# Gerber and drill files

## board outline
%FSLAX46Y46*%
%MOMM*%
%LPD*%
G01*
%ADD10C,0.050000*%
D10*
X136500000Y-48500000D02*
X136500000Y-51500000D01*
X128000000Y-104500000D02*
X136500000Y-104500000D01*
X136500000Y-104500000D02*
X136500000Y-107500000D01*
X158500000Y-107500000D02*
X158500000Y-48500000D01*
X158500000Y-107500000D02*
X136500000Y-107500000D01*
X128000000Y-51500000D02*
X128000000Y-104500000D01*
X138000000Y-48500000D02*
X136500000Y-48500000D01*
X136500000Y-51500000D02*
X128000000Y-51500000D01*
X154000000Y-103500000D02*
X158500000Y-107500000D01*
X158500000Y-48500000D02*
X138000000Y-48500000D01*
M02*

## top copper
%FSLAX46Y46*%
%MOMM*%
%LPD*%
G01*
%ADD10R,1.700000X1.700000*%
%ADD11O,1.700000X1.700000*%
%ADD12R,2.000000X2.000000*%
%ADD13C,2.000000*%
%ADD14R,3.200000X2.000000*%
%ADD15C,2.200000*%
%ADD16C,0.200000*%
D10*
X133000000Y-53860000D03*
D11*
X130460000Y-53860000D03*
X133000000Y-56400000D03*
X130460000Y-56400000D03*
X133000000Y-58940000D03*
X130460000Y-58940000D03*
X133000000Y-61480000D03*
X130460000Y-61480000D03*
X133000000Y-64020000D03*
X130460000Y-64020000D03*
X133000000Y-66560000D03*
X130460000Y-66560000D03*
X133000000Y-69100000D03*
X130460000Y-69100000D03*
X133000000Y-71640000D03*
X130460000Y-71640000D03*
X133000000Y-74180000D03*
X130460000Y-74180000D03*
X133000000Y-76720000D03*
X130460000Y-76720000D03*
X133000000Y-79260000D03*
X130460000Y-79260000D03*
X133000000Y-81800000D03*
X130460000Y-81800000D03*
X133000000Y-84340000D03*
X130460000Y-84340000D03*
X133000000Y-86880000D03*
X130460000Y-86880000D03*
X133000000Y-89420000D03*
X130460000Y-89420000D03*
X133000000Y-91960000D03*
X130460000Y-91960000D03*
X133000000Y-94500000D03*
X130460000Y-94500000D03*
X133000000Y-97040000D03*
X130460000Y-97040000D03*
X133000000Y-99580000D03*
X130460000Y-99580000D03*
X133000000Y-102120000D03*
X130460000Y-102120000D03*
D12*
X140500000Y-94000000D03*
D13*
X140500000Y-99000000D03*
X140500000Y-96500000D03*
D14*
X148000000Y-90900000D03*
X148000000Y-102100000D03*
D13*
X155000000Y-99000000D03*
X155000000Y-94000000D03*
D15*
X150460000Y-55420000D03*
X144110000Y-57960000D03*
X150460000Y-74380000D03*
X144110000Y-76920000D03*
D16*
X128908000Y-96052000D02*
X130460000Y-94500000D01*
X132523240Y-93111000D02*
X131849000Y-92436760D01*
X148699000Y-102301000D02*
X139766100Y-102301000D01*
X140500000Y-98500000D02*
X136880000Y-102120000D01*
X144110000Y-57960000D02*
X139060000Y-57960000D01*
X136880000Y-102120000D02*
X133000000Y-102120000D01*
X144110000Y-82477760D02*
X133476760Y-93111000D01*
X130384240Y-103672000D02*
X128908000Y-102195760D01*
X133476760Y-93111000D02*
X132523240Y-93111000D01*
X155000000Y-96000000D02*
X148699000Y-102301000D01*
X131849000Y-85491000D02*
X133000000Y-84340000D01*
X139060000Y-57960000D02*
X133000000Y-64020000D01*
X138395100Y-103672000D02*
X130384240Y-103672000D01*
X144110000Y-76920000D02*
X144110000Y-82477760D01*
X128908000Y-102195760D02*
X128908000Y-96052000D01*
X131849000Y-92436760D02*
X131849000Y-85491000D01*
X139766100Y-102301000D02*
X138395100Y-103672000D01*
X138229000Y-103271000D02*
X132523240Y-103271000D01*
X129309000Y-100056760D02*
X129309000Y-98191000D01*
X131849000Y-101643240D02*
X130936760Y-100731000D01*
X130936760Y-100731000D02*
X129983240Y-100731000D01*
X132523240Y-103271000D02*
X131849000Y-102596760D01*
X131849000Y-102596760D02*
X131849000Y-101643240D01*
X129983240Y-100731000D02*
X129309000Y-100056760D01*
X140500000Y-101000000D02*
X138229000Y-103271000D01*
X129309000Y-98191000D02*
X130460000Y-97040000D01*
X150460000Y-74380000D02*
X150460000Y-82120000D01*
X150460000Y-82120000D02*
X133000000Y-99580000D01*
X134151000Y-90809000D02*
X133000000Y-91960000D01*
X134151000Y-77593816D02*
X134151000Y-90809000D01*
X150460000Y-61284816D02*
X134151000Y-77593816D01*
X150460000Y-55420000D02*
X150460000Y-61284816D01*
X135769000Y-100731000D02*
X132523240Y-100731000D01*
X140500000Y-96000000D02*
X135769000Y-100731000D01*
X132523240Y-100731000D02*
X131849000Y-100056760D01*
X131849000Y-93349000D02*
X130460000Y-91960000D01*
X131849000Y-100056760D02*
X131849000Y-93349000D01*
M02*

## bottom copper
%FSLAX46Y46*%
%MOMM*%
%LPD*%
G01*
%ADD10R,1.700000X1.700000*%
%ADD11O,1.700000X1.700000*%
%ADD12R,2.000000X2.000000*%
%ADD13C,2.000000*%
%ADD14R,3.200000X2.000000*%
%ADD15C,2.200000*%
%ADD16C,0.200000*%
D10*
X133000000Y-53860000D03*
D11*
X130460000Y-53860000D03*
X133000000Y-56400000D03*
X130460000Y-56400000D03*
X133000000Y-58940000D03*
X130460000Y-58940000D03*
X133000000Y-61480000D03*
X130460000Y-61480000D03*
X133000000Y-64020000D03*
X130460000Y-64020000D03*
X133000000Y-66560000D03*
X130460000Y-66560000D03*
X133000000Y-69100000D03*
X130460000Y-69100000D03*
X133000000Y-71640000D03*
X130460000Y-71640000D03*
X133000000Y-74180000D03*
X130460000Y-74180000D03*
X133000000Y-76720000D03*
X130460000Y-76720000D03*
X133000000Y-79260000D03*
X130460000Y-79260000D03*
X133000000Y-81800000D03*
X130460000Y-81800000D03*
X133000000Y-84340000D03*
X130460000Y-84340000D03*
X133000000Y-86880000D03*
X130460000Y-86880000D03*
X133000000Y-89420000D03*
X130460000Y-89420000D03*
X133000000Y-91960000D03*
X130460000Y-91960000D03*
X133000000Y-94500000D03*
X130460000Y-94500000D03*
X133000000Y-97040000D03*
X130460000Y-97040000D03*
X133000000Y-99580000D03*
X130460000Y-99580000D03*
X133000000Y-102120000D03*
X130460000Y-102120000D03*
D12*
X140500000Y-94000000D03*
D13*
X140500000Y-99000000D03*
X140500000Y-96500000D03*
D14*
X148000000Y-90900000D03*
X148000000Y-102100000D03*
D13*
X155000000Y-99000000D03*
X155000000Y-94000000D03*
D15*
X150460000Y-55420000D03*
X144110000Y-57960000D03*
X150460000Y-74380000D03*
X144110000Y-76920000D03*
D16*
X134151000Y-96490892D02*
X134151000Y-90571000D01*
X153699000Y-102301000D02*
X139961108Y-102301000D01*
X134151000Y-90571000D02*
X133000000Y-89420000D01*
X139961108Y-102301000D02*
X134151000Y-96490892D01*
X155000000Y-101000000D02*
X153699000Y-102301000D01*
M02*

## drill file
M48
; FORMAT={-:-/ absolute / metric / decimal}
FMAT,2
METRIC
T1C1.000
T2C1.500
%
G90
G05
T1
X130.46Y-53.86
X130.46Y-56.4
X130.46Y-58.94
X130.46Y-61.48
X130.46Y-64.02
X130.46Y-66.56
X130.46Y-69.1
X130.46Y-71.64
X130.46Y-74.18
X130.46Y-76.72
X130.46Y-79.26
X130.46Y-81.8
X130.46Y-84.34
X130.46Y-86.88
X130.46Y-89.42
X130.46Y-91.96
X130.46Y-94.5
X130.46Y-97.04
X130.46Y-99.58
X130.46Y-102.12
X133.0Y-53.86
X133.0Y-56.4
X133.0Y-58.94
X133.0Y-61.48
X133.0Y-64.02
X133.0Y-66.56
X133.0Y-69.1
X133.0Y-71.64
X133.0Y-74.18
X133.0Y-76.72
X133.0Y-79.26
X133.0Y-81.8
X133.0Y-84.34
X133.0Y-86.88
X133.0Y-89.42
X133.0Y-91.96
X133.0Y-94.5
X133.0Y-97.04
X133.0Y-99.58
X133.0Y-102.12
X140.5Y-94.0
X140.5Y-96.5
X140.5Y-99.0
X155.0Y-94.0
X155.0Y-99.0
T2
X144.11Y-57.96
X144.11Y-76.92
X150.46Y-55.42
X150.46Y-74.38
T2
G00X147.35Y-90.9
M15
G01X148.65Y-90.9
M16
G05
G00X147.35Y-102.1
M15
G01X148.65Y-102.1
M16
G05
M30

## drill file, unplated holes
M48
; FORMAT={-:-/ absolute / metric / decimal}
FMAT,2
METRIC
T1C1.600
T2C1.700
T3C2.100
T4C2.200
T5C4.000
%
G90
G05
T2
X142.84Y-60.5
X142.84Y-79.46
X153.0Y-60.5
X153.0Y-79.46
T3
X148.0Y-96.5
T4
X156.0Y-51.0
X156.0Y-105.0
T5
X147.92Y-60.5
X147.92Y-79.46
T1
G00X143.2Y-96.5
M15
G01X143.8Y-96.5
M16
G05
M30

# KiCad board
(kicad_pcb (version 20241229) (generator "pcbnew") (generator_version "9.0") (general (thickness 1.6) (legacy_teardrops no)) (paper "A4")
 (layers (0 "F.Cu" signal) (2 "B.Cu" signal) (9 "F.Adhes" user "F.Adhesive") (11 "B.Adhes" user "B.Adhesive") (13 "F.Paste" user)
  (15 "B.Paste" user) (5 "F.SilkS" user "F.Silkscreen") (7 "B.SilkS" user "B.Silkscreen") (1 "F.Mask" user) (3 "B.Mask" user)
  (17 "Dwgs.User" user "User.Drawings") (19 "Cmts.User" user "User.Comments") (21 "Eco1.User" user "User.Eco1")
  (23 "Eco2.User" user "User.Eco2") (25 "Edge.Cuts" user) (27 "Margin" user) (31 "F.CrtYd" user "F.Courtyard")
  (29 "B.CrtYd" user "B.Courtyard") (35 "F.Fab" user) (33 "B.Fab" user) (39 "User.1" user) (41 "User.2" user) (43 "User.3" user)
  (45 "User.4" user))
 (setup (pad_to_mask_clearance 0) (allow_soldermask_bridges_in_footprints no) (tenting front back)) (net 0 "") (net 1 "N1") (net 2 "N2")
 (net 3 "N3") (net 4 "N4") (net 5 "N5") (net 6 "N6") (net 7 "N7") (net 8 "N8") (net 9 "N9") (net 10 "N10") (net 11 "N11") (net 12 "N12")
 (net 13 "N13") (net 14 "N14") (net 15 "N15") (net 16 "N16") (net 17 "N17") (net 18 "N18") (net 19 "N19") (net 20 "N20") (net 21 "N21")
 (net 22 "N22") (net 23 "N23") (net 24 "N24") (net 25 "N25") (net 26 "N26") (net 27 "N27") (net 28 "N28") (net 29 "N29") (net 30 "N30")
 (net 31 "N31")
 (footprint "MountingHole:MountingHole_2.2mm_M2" (layer "F.Cu") (at 156 105)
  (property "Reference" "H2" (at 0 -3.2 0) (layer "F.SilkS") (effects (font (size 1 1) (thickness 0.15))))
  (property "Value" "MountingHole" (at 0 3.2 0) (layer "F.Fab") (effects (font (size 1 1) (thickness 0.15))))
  (pad "" np_thru_hole circle (at 0 0) (size 2.2 2.2) (drill 2.2) (layers "*.Cu" "*.Mask")))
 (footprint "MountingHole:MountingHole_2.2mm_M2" (layer "F.Cu") (at 156 51)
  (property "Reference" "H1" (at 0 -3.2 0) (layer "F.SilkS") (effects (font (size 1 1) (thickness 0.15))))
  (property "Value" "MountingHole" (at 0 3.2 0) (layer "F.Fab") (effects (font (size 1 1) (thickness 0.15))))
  (pad "" np_thru_hole circle (at 0 0) (size 2.2 2.2) (drill 2.2) (layers "*.Cu" "*.Mask")))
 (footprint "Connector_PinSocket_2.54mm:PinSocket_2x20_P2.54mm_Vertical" (layer "F.Cu") (at 133 53.86)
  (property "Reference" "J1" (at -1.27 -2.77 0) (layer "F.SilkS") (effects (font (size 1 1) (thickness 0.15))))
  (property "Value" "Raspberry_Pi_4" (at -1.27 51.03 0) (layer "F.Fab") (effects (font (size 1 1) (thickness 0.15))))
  (pad "1" thru_hole rect (at 0 0) (size 1.7 1.7) (drill 1) (layers "*.Cu" "*.Mask") (remove_unused_layers no) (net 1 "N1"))
  (pad "2" thru_hole oval (at -2.54 0) (size 1.7 1.7) (drill 1) (layers "*.Cu" "*.Mask") (remove_unused_layers no) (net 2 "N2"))
  (pad "3" thru_hole oval (at 0 2.54) (size 1.7 1.7) (drill 1) (layers "*.Cu" "*.Mask") (remove_unused_layers no) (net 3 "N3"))
  (pad "4" thru_hole oval (at -2.54 2.54) (size 1.7 1.7) (drill 1) (layers "*.Cu" "*.Mask") (remove_unused_layers no) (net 2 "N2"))
  (pad "5" thru_hole oval (at 0 5.08) (size 1.7 1.7) (drill 1) (layers "*.Cu" "*.Mask") (remove_unused_layers no) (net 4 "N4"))
  (pad "6" thru_hole oval (at -2.54 5.08) (size 1.7 1.7) (drill 1) (layers "*.Cu" "*.Mask") (remove_unused_layers no) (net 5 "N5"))
  (pad "7" thru_hole oval (at 0 7.62) (size 1.7 1.7) (drill 1) (layers "*.Cu" "*.Mask") (remove_unused_layers no) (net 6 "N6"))
  (pad "8" thru_hole oval (at -2.54 7.62) (size 1.7 1.7) (drill 1) (layers "*.Cu" "*.Mask") (remove_unused_layers no) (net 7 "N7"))
  (pad "9" thru_hole oval (at 0 10.16) (size 1.7 1.7) (drill 1) (layers "*.Cu" "*.Mask") (remove_unused_layers no) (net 5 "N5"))
  (pad "10" thru_hole oval (at -2.54 10.16) (size 1.7 1.7) (drill 1) (layers "*.Cu" "*.Mask") (remove_unused_layers no) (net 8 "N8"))
  (pad "11" thru_hole oval (at 0 12.7) (size 1.7 1.7) (drill 1) (layers "*.Cu" "*.Mask") (remove_unused_layers no) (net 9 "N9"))
  (pad "12" thru_hole oval (at -2.54 12.7) (size 1.7 1.7) (drill 1) (layers "*.Cu" "*.Mask") (remove_unused_layers no) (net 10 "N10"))
  (pad "13" thru_hole oval (at 0 15.24) (size 1.7 1.7) (drill 1) (layers "*.Cu" "*.Mask") (remove_unused_layers no) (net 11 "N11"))
  (pad "14" thru_hole oval (at -2.54 15.24) (size 1.7 1.7) (drill 1) (layers "*.Cu" "*.Mask") (remove_unused_layers no) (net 5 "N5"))
  (pad "15" thru_hole oval (at 0 17.78) (size 1.7 1.7) (drill 1) (layers "*.Cu" "*.Mask") (remove_unused_layers no) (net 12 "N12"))
  (pad "16" thru_hole oval (at -2.54 17.78) (size 1.7 1.7) (drill 1) (layers "*.Cu" "*.Mask") (remove_unused_layers no) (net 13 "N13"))
  (pad "17" thru_hole oval (at 0 20.32) (size 1.7 1.7) (drill 1) (layers "*.Cu" "*.Mask") (remove_unused_layers no) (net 1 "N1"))
  (pad "18" thru_hole oval (at -2.54 20.32) (size 1.7 1.7) (drill 1) (layers "*.Cu" "*.Mask") (remove_unused_layers no) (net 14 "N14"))
  (pad "19" thru_hole oval (at 0 22.86) (size 1.7 1.7) (drill 1) (layers "*.Cu" "*.Mask") (remove_unused_layers no) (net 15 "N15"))
  (pad "20" thru_hole oval (at -2.54 22.86) (size 1.7 1.7) (drill 1) (layers "*.Cu" "*.Mask") (remove_unused_layers no) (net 5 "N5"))
  (pad "21" thru_hole oval (at 0 25.4) (size 1.7 1.7) (drill 1) (layers "*.Cu" "*.Mask") (remove_unused_layers no) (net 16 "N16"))
  (pad "22" thru_hole oval (at -2.54 25.4) (size 1.7 1.7) (drill 1) (layers "*.Cu" "*.Mask") (remove_unused_layers no) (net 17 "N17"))
  (pad "23" thru_hole oval (at 0 27.94) (size 1.7 1.7) (drill 1) (layers "*.Cu" "*.Mask") (remove_unused_layers no) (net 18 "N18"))
  (pad "24" thru_hole oval (at -2.54 27.94) (size 1.7 1.7) (drill 1) (layers "*.Cu" "*.Mask") (remove_unused_layers no) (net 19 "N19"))
  (pad "25" thru_hole oval (at 0 30.48) (size 1.7 1.7) (drill 1) (layers "*.Cu" "*.Mask") (remove_unused_layers no) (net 5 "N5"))
  (pad "26" thru_hole oval (at -2.54 30.48) (size 1.7 1.7) (drill 1) (layers "*.Cu" "*.Mask") (remove_unused_layers no) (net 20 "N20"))
  (pad "27" thru_hole oval (at 0 33.02) (size 1.7 1.7) (drill 1) (layers "*.Cu" "*.Mask") (remove_unused_layers no) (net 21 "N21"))
  (pad "28" thru_hole oval (at -2.54 33.02) (size 1.7 1.7) (drill 1) (layers "*.Cu" "*.Mask") (remove_unused_layers no) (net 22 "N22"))
  (pad "29" thru_hole oval (at 0 35.56) (size 1.7 1.7) (drill 1) (layers "*.Cu" "*.Mask") (remove_unused_layers no) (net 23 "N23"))
  (pad "30" thru_hole oval (at -2.54 35.56) (size 1.7 1.7) (drill 1) (layers "*.Cu" "*.Mask") (remove_unused_layers no) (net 5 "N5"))
  (pad "31" thru_hole oval (at 0 38.1) (size 1.7 1.7) (drill 1) (layers "*.Cu" "*.Mask") (remove_unused_layers no) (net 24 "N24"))
  (pad "32" thru_hole oval (at -2.54 38.1) (size 1.7 1.7) (drill 1) (layers "*.Cu" "*.Mask") (remove_unused_layers no) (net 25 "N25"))
  (pad "33" thru_hole oval (at 0 40.64) (size 1.7 1.7) (drill 1) (layers "*.Cu" "*.Mask") (remove_unused_layers no) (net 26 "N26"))
  (pad "34" thru_hole oval (at -2.54 40.64) (size 1.7 1.7) (drill 1) (layers "*.Cu" "*.Mask") (remove_unused_layers no) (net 5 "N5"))
  (pad "35" thru_hole oval (at 0 43.18) (size 1.7 1.7) (drill 1) (layers "*.Cu" "*.Mask") (remove_unused_layers no) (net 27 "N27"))
  (pad "36" thru_hole oval (at -2.54 43.18) (size 1.7 1.7) (drill 1) (layers "*.Cu" "*.Mask") (remove_unused_layers no) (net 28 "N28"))
  (pad "37" thru_hole oval (at 0 45.72) (size 1.7 1.7) (drill 1) (layers "*.Cu" "*.Mask") (remove_unused_layers no) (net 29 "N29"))
  (pad "38" thru_hole oval (at -2.54 45.72) (size 1.7 1.7) (drill 1) (layers "*.Cu" "*.Mask") (remove_unused_layers no) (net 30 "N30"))
  (pad "39" thru_hole oval (at 0 48.26) (size 1.7 1.7) (drill 1) (layers "*.Cu" "*.Mask") (remove_unused_layers no) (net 5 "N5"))
  (pad "40" thru_hole oval (at -2.54 48.26) (size 1.7 1.7) (drill 1) (layers "*.Cu" "*.Mask") (remove_unused_layers no) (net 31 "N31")))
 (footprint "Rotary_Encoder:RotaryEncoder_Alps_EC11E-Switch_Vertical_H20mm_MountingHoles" (layer "F.Cu") (at 140.5 94)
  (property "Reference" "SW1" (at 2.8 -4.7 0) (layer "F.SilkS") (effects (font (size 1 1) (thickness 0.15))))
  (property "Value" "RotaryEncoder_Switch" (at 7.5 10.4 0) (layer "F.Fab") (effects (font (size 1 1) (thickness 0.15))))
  (pad "" np_thru_hole oval (at 3 2.5) (size 2.2 1.6) (drill oval 2.2 1.6) (layers "*.Mask"))
  (pad "" np_thru_hole circle (at 7.5 2.5) (size 2.1 2.1) (drill 2.1) (layers "*.Mask"))
  (pad "A" thru_hole rect (at 0 0) (size 2 2) (drill 1) (layers "*.Cu" "*.Mask") (remove_unused_layers no) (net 25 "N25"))
  (pad "B" thru_hole circle (at 0 5) (size 2 2) (drill 1) (layers "*.Cu" "*.Mask") (remove_unused_layers no) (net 28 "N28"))
  (pad "C" thru_hole circle (at 0 2.5) (size 2 2) (drill 1) (layers "*.Cu" "*.Mask") (remove_unused_layers no) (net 5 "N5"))
  (pad "MP" thru_hole rect (at 7.5 -3.1) (size 3.2 2) (drill oval 2.8 1.5) (layers "*.Cu" "*.Mask") (remove_unused_layers no))
  (pad "MP" thru_hole rect (at 7.5 8.1) (size 3.2 2) (drill oval 2.8 1.5) (layers "*.Cu" "*.Mask") (remove_unused_layers no))
  (pad "S1" thru_hole circle (at 14.5 5) (size 2 2) (drill 1) (layers "*.Cu" "*.Mask") (remove_unused_layers no) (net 23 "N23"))
  (pad "S2" thru_hole circle (at 14.5 0) (size 2 2) (drill 1) (layers "*.Cu" "*.Mask") (remove_unused_layers no) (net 5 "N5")))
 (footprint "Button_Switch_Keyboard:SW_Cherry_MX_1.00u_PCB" (layer "F.Cu") (at 150.46 55.42)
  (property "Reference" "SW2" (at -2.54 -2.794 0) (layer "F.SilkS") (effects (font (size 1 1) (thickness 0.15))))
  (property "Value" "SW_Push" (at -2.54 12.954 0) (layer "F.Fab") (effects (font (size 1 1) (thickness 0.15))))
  (pad "" np_thru_hole circle (at -7.62 5.08) (size 1.7 1.7) (drill 1.7) (layers "*.Cu" "*.Mask"))
  (pad "" np_thru_hole circle (at -2.54 5.08) (size 4 4) (drill 4) (layers "*.Cu" "*.Mask"))
  (pad "" np_thru_hole circle (at 2.54 5.08) (size 1.7 1.7) (drill 1.7) (layers "*.Cu" "*.Mask"))
  (pad "1" thru_hole circle (at 0 0) (size 2.2 2.2) (drill 1.5) (layers "*.Cu" "*.Mask") (remove_unused_layers no) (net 24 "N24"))
  (pad "2" thru_hole circle (at -6.35 2.54) (size 2.2 2.2) (drill 1.5) (layers "*.Cu" "*.Mask") (remove_unused_layers no) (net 5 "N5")))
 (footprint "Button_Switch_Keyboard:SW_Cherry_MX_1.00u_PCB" (layer "F.Cu") (at 150.46 74.38)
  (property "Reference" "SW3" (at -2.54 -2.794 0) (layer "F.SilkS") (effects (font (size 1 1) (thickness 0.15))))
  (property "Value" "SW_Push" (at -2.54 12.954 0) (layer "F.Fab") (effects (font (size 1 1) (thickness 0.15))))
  (pad "" np_thru_hole circle (at -7.62 5.08) (size 1.7 1.7) (drill 1.7) (layers "*.Cu" "*.Mask"))
  (pad "" np_thru_hole circle (at -2.54 5.08) (size 4 4) (drill 4) (layers "*.Cu" "*.Mask"))
  (pad "" np_thru_hole circle (at 2.54 5.08) (size 1.7 1.7) (drill 1.7) (layers "*.Cu" "*.Mask"))
  (pad "1" thru_hole circle (at 0 0) (size 2.2 2.2) (drill 1.5) (layers "*.Cu" "*.Mask") (remove_unused_layers no) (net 29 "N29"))
  (pad "2" thru_hole circle (at -6.35 2.54) (size 2.2 2.2) (drill 1.5) (layers "*.Cu" "*.Mask") (remove_unused_layers no) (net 5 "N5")))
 (gr_line (start 136.5 48.5) (end 136.5 51.5) (stroke (width 0.05) (type default)) (layer "Edge.Cuts"))
 (gr_line (start 128 104.5) (end 136.5 104.5) (stroke (width 0.05) (type default)) (layer "Edge.Cuts"))
 (gr_line (start 136.5 104.5) (end 136.5 107.5) (stroke (width 0.05) (type default)) (layer "Edge.Cuts"))
 (gr_line (start 158.5 107.5) (end 158.5 48.5) (stroke (width 0.05) (type default)) (layer "Edge.Cuts"))
 (gr_line (start 158.5 107.5) (end 136.5 107.5) (stroke (width 0.05) (type default)) (layer "Edge.Cuts"))
 (gr_line (start 128 51.5) (end 128 104.5) (stroke (width 0.05) (type default)) (layer "Edge.Cuts"))
 (gr_line (start 138 48.5) (end 136.5 48.5) (stroke (width 0.05) (type default)) (layer "Edge.Cuts"))
 (gr_line (start 136.5 51.5) (end 128 51.5) (stroke (width 0.05) (type default)) (layer "Edge.Cuts"))
 (gr_line (start 154 103.5) (end 158.5 107.5) (stroke (width 0.05) (type default)) (layer "Edge.Cuts"))
 (gr_line (start 158.5 48.5) (end 138 48.5) (stroke (width 0.05) (type default)) (layer "Edge.Cuts"))
 (segment (start 134.151 96.490892) (end 134.151 90.571) (width 0.2) (layer "B.Cu") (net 23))
 (segment (start 153.699 102.301) (end 139.961108 102.301) (width 0.2) (layer "B.Cu") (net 23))
 (segment (start 134.151 90.571) (end 133 89.42) (width 0.2) (layer "B.Cu") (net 23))
 (segment (start 139.961108 102.301) (end 134.151 96.490892) (width 0.2) (layer "B.Cu") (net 23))
 (segment (start 155 101) (end 153.699 102.301) (width 0.2) (layer "B.Cu") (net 23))
 (segment (start 128.908 96.052) (end 130.46 94.5) (width 0.2) (layer "F.Cu") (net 5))
 (segment (start 132.52324 93.111) (end 131.849 92.43676) (width 0.2) (layer "F.Cu") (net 5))
 (segment (start 148.699 102.301) (end 139.7661 102.301) (width 0.2) (layer "F.Cu") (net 5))
 (segment (start 140.5 98.5) (end 136.88 102.12) (width 0.2) (layer "F.Cu") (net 5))
 (segment (start 144.11 57.96) (end 139.06 57.96) (width 0.2) (layer "F.Cu") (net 5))
 (segment (start 136.88 102.12) (end 133 102.12) (width 0.2) (layer "F.Cu") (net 5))
 (segment (start 144.11 82.47776) (end 133.47676 93.111) (width 0.2) (layer "F.Cu") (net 5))
 (segment (start 130.38424 103.672) (end 128.908 102.19576) (width 0.2) (layer "F.Cu") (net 5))
 (segment (start 133.47676 93.111) (end 132.52324 93.111) (width 0.2) (layer "F.Cu") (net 5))
 (segment (start 155 96) (end 148.699 102.301) (width 0.2) (layer "F.Cu") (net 5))
 (segment (start 131.849 85.491) (end 133 84.34) (width 0.2) (layer "F.Cu") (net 5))
 (segment (start 139.06 57.96) (end 133 64.02) (width 0.2) (layer "F.Cu") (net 5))
 (segment (start 138.3951 103.672) (end 130.38424 103.672) (width 0.2) (layer "F.Cu") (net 5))
 (segment (start 144.11 76.92) (end 144.11 82.47776) (width 0.2) (layer "F.Cu") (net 5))
 (segment (start 128.908 102.19576) (end 128.908 96.052) (width 0.2) (layer "F.Cu") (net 5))
 (segment (start 131.849 92.43676) (end 131.849 85.491) (width 0.2) (layer "F.Cu") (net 5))
 (segment (start 139.7661 102.301) (end 138.3951 103.672) (width 0.2) (layer "F.Cu") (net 5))
 (segment (start 138.229 103.271) (end 132.52324 103.271) (width 0.2) (layer "F.Cu") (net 28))
 (segment (start 129.309 100.05676) (end 129.309 98.191) (width 0.2) (layer "F.Cu") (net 28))
 (segment (start 131.849 101.64324) (end 130.93676 100.731) (width 0.2) (layer "F.Cu") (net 28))
 (segment (start 130.93676 100.731) (end 129.98324 100.731) (width 0.2) (layer "F.Cu") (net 28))
 (segment (start 132.52324 103.271) (end 131.849 102.59676) (width 0.2) (layer "F.Cu") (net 28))
 (segment (start 131.849 102.59676) (end 131.849 101.64324) (width 0.2) (layer "F.Cu") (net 28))
 (segment (start 129.98324 100.731) (end 129.309 100.05676) (width 0.2) (layer "F.Cu") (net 28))
 (segment (start 140.5 101) (end 138.229 103.271) (width 0.2) (layer "F.Cu") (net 28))
 (segment (start 129.309 98.191) (end 130.46 97.04) (width 0.2) (layer "F.Cu") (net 28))
 (segment (start 150.46 74.38) (end 150.46 82.12) (width 0.2) (layer "F.Cu") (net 29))
 (segment (start 150.46 82.12) (end 133 99.58) (width 0.2) (layer "F.Cu") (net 29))
 (segment (start 134.151 90.809) (end 133 91.96) (width 0.2) (layer "F.Cu") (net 24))
 (segment (start 134.151 77.593816) (end 134.151 90.809) (width 0.2) (layer "F.Cu") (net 24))
 (segment (start 150.46 61.284816) (end 134.151 77.593816) (width 0.2) (layer "F.Cu") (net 24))
 (segment (start 150.46 55.42) (end 150.46 61.284816) (width 0.2) (layer "F.Cu") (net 24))
 (segment (start 135.769 100.731) (end 132.52324 100.731) (width 0.2) (layer "F.Cu") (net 25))
 (segment (start 140.5 96) (end 135.769 100.731) (width 0.2) (layer "F.Cu") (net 25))
 (segment (start 132.52324 100.731) (end 131.849 100.05676) (width 0.2) (layer "F.Cu") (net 25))
 (segment (start 131.849 93.349) (end 130.46 91.96) (width 0.2) (layer "F.Cu") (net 25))
 (segment (start 131.849 100.05676) (end 131.849 93.349) (width 0.2) (layer "F.Cu") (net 25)))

